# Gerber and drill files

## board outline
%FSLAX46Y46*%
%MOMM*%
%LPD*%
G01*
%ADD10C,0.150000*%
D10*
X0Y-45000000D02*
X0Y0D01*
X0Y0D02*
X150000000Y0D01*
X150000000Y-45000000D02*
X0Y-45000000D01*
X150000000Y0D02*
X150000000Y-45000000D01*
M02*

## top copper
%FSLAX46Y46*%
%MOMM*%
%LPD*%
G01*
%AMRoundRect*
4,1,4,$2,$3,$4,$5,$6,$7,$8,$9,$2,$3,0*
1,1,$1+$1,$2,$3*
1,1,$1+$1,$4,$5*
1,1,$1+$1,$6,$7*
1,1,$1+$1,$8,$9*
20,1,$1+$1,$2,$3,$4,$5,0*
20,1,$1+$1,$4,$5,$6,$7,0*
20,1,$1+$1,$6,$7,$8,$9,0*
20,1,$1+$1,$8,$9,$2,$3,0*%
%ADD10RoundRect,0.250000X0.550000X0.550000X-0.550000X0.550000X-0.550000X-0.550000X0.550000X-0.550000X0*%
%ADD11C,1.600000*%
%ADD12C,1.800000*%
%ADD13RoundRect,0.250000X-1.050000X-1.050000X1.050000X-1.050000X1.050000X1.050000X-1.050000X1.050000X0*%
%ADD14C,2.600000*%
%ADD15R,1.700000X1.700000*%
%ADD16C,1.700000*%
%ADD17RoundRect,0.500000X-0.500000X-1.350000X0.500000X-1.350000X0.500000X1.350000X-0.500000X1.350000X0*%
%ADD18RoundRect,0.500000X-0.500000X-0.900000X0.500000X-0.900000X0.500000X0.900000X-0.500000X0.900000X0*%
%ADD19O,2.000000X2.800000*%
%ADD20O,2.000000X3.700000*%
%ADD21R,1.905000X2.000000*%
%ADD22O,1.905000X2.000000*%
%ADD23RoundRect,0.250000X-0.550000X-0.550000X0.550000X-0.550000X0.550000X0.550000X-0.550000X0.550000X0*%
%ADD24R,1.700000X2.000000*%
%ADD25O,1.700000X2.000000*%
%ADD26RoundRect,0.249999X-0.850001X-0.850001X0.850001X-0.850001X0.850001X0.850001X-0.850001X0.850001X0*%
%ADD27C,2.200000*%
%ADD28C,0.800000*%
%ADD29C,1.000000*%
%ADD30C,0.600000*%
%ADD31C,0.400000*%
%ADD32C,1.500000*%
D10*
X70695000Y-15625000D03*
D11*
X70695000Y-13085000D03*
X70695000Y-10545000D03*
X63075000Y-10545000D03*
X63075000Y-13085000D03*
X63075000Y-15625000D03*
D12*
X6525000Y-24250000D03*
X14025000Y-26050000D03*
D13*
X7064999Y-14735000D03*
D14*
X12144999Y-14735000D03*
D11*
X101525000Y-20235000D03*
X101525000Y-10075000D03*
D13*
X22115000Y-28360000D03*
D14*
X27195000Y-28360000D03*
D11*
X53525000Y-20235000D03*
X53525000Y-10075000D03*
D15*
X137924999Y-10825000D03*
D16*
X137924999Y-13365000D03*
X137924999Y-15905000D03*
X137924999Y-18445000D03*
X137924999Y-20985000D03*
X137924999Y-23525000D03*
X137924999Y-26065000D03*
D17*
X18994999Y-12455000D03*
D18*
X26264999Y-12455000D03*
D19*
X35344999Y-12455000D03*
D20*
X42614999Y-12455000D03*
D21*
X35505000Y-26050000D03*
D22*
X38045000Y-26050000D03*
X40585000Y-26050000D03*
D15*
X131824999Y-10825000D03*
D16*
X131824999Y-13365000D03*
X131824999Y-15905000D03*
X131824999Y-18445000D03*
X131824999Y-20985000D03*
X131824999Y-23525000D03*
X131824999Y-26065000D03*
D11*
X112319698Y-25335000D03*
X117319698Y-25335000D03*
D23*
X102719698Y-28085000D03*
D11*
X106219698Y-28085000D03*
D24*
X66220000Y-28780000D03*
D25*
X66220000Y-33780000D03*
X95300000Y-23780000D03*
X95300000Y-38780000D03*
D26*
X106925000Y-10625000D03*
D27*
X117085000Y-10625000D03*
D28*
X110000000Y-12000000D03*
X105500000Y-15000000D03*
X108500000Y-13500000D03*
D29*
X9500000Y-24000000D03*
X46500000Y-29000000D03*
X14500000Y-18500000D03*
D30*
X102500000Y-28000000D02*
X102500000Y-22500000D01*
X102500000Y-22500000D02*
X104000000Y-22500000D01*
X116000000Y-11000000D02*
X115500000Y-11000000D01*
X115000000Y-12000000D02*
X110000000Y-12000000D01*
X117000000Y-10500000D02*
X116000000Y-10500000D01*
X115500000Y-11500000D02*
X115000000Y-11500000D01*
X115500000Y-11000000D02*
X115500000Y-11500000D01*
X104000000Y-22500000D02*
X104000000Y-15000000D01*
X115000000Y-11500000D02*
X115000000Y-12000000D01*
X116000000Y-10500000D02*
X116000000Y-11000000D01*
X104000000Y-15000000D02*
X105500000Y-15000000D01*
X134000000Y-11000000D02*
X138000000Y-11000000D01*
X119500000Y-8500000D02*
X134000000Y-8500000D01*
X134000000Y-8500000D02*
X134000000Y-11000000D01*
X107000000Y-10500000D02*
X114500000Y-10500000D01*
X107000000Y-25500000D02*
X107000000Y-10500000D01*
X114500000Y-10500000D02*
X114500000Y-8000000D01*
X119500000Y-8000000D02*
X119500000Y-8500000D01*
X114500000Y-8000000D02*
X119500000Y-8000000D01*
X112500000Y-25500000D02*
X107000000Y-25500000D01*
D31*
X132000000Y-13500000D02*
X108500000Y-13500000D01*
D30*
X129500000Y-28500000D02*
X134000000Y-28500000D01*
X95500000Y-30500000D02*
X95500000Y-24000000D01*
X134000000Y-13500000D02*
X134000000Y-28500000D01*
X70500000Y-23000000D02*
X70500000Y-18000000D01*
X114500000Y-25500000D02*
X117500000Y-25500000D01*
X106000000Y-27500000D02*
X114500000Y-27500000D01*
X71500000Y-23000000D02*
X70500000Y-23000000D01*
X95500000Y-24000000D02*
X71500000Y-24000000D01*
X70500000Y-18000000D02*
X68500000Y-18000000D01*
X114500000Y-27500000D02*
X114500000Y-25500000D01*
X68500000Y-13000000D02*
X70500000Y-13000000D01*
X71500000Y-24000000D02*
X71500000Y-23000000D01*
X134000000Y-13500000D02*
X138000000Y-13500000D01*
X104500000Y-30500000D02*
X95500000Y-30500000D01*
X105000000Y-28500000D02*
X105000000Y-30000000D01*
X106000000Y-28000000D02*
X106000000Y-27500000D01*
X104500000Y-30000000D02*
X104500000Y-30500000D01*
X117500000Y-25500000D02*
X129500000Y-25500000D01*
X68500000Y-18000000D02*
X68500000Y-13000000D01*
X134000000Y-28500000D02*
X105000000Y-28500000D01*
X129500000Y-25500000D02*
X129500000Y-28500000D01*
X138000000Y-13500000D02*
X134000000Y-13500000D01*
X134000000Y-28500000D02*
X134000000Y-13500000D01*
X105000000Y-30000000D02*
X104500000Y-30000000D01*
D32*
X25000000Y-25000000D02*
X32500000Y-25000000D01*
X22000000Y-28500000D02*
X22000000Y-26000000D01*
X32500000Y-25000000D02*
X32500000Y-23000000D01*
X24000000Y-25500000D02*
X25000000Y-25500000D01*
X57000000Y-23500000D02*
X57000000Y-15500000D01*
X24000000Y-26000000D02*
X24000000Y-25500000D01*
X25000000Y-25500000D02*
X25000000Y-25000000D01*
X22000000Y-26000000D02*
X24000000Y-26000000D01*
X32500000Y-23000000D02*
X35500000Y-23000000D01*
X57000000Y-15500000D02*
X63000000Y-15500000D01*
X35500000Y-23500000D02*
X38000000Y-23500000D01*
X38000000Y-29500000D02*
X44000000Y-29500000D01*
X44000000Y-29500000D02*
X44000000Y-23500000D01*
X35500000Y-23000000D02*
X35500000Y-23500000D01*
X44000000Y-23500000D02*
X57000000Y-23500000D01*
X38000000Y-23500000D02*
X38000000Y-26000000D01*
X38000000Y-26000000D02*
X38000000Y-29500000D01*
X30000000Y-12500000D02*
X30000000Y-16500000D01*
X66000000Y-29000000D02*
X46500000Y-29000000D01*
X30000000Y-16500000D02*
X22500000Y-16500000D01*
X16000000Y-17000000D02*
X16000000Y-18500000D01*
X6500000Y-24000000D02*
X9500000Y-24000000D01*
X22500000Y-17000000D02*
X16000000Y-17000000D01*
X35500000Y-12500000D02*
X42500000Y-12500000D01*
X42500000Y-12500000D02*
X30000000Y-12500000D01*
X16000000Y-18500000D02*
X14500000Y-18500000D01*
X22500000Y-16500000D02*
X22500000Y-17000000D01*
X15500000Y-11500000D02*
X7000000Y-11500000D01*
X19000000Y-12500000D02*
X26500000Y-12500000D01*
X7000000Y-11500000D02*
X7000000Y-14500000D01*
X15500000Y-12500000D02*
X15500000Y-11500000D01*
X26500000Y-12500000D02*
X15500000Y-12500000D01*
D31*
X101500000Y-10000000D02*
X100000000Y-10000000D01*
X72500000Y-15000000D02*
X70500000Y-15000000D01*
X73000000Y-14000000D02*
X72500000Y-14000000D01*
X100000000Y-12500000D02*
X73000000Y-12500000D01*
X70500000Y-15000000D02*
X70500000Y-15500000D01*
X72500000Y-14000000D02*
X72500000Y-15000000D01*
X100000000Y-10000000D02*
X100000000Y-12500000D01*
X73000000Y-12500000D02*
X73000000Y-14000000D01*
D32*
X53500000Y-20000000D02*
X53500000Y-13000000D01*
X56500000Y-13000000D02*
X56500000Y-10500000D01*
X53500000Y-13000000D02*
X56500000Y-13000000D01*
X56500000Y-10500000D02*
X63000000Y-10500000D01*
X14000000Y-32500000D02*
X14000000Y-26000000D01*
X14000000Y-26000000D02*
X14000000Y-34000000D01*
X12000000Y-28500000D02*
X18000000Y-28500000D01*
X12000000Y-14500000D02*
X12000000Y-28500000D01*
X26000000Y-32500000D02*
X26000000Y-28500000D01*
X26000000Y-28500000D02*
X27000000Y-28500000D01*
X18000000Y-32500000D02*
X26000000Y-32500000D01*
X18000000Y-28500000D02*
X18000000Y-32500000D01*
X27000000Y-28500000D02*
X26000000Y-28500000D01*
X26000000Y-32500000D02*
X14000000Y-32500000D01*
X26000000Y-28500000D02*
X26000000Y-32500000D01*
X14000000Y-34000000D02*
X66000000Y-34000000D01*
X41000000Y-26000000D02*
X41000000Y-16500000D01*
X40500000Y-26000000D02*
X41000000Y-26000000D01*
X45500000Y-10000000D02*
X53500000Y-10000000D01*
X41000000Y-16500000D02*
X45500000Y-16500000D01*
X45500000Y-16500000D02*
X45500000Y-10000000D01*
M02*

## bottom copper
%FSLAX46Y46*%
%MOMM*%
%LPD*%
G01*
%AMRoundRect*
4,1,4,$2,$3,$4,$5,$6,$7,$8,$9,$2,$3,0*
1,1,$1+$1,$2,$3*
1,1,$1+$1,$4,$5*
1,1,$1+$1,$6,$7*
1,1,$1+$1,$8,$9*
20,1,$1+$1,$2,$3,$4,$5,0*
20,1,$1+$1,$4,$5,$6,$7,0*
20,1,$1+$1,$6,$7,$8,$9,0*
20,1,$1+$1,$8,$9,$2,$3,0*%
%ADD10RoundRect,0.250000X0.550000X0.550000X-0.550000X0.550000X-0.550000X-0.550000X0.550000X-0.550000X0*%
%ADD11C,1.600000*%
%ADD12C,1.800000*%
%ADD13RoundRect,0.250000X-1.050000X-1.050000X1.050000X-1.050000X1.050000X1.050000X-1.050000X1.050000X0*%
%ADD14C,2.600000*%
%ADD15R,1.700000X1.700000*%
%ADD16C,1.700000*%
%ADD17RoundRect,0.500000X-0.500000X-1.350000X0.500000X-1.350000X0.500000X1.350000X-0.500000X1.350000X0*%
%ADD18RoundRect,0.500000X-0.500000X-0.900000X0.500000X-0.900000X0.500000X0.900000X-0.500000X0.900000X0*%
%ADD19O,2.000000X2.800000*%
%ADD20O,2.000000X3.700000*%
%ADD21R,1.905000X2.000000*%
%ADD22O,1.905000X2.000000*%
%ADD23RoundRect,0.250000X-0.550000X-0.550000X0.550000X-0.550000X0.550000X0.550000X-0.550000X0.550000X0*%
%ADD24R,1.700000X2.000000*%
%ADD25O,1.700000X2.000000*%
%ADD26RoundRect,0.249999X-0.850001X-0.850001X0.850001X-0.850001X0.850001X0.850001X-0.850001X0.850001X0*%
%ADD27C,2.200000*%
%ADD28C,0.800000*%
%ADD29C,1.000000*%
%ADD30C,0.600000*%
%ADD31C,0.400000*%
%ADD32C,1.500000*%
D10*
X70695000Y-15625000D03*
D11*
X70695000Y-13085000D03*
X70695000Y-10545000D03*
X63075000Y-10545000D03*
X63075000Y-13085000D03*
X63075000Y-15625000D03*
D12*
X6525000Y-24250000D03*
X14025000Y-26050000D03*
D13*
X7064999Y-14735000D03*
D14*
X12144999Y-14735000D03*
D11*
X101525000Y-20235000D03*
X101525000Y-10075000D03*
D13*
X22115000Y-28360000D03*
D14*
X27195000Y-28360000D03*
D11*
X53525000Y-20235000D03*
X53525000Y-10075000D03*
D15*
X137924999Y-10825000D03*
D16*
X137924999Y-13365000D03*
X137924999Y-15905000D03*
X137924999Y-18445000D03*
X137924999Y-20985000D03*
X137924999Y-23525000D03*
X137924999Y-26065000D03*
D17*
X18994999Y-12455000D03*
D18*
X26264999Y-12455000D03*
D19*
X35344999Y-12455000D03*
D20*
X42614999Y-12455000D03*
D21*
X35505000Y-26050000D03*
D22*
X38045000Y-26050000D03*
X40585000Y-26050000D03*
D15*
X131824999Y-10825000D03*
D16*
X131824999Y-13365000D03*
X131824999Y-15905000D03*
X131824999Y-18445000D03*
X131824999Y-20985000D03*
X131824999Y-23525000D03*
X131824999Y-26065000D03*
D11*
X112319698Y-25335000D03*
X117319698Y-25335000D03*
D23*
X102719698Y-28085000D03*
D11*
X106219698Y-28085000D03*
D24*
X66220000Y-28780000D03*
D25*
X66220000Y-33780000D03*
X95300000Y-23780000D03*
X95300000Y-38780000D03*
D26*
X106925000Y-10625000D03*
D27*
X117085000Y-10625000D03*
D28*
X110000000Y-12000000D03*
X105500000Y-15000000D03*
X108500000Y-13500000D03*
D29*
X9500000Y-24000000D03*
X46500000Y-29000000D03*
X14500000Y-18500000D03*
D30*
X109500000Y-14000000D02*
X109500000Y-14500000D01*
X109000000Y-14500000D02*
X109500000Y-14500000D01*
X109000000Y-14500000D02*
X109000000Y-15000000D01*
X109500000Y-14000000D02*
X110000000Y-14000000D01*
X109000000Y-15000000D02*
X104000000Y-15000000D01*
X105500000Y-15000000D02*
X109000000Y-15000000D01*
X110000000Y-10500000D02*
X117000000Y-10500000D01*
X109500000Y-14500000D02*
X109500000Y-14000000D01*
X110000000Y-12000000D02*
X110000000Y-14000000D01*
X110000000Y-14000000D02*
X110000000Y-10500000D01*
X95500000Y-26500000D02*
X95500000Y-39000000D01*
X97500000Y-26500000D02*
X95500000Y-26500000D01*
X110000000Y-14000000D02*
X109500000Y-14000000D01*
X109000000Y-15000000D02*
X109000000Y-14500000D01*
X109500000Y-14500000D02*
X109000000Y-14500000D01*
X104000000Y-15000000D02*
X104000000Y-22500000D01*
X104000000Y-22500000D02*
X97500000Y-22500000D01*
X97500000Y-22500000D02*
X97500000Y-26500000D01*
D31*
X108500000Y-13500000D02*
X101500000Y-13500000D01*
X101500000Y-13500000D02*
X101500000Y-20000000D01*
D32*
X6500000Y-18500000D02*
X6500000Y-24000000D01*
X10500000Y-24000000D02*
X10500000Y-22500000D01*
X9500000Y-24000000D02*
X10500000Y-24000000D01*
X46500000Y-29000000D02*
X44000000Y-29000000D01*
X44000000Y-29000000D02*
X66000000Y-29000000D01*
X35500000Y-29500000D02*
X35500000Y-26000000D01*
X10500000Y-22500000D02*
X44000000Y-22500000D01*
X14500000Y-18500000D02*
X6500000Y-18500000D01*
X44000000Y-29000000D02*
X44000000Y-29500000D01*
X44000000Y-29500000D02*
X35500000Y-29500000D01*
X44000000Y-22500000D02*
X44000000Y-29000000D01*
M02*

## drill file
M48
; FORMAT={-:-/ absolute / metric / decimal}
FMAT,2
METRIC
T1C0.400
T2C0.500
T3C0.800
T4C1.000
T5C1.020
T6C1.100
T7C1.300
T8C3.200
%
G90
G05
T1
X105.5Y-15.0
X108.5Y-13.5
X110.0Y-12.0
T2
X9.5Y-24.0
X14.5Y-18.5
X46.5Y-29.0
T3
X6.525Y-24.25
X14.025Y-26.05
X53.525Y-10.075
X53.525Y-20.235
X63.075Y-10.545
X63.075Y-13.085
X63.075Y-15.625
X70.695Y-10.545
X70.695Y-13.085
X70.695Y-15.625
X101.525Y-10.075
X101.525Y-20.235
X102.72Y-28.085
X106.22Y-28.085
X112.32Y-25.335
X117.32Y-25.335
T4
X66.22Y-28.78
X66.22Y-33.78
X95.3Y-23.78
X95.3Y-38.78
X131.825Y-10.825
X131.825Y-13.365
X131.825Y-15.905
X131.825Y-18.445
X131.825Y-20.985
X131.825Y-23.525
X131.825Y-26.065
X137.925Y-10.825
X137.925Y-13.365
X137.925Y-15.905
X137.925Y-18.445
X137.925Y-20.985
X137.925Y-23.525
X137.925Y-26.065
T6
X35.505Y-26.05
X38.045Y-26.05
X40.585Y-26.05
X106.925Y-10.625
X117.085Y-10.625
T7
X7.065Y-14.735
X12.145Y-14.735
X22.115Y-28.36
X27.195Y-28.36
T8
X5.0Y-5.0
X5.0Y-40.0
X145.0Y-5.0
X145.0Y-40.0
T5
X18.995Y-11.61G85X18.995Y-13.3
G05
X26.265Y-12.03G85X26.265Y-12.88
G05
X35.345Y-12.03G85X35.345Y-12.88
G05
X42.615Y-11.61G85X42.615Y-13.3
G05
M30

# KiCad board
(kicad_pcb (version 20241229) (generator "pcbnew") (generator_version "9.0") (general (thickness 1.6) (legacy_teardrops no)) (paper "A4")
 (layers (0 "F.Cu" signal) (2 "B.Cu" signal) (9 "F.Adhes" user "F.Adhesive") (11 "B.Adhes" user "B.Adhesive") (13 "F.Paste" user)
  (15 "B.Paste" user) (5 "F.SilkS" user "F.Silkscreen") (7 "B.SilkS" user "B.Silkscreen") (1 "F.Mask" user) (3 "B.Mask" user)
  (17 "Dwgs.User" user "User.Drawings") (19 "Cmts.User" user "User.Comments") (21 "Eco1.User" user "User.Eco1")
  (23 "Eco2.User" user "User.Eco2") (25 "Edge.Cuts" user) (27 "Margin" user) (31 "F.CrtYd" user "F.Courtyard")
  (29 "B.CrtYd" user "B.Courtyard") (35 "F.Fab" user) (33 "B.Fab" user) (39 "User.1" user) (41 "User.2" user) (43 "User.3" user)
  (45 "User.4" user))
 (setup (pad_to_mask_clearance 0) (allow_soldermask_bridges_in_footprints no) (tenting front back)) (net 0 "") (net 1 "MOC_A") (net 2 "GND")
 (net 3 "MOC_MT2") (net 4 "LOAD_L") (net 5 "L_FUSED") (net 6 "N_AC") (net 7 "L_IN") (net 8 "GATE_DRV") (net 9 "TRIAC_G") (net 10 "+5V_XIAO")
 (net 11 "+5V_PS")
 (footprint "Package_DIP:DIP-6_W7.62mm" (layer "F.Cu") (at 70.695 15.625 180)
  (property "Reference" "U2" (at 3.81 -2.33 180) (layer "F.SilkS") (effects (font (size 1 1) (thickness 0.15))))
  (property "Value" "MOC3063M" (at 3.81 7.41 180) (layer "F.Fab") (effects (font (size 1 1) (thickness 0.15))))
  (pad "1" thru_hole roundrect (at 0 0 180) (size 1.6 1.6) (drill 0.8) (layers "*.Cu" "*.Mask") (remove_unused_layers no)
   (roundrect_rratio 0.15625) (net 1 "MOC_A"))
  (pad "2" thru_hole circle (at 0 2.54 180) (size 1.6 1.6) (drill 0.8) (layers "*.Cu" "*.Mask") (remove_unused_layers no) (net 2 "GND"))
  (pad "3" thru_hole circle (at 0 5.08 180) (size 1.6 1.6) (drill 0.8) (layers "*.Cu" "*.Mask") (remove_unused_layers no))
  (pad "4" thru_hole circle (at 7.62 5.08 180) (size 1.6 1.6) (drill 0.8) (layers "*.Cu" "*.Mask") (remove_unused_layers no)
   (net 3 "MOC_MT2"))
  (pad "5" thru_hole circle (at 7.62 2.54 180) (size 1.6 1.6) (drill 0.8) (layers "*.Cu" "*.Mask") (remove_unused_layers no))
  (pad "6" thru_hole circle (at 7.62 0 180) (size 1.6 1.6) (drill 0.8) (layers "*.Cu" "*.Mask") (remove_unused_layers no) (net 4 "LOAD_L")))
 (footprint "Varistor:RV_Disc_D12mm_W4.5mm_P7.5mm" (layer "F.Cu") (at 6.525 24.25)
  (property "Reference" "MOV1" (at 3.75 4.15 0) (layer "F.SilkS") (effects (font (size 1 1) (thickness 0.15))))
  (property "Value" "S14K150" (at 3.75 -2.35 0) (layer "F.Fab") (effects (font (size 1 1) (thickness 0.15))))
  (pad "1" thru_hole circle (at 0 0) (size 1.8 1.8) (drill 0.8) (layers "*.Cu" "*.Mask") (remove_unused_layers no) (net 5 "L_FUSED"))
  (pad "2" thru_hole circle (at 7.5 1.8) (size 1.8 1.8) (drill 0.8) (layers "*.Cu" "*.Mask") (remove_unused_layers no) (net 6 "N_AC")))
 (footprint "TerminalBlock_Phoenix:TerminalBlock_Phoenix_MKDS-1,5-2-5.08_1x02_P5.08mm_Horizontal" (layer "F.Cu") (at 7.064999 14.735)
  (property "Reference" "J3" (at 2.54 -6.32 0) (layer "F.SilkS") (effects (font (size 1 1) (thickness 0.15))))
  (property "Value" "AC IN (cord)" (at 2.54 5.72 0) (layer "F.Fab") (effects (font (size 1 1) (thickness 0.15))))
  (pad "1" thru_hole roundrect (at 0 0) (size 2.6 2.6) (drill 1.3) (layers "*.Cu" "*.Mask") (remove_unused_layers no)
   (roundrect_rratio 0.096154) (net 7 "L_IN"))
  (pad "2" thru_hole circle (at 5.08 0) (size 2.6 2.6) (drill 1.3) (layers "*.Cu" "*.Mask") (remove_unused_layers no) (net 6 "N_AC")))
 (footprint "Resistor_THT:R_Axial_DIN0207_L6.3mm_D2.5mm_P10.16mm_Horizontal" (layer "F.Cu") (at 101.525 20.235 90)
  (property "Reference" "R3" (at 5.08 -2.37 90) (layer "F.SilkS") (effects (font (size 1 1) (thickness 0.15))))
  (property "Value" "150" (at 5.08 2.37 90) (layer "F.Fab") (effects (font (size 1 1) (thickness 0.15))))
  (pad "1" thru_hole circle (at 0 0 90) (size 1.6 1.6) (drill 0.8) (layers "*.Cu" "*.Mask") (remove_unused_layers no) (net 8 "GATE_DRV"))
  (pad "2" thru_hole circle (at 10.16 0 90) (size 1.6 1.6) (drill 0.8) (layers "*.Cu" "*.Mask") (remove_unused_layers no) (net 1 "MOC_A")))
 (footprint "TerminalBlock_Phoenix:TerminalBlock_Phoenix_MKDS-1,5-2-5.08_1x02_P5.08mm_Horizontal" (layer "F.Cu") (at 22.115 28.36)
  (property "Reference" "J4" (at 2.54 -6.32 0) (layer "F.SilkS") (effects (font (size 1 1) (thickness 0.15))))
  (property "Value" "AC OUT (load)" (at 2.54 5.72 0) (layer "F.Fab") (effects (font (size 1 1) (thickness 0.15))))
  (pad "1" thru_hole roundrect (at 0 0) (size 2.6 2.6) (drill 1.3) (layers "*.Cu" "*.Mask") (remove_unused_layers no)
   (roundrect_rratio 0.096154) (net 4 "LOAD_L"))
  (pad "2" thru_hole circle (at 5.08 0) (size 2.6 2.6) (drill 1.3) (layers "*.Cu" "*.Mask") (remove_unused_layers no) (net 6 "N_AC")))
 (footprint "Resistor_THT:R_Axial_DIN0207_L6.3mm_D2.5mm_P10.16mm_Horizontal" (layer "F.Cu") (at 53.525 20.235 90)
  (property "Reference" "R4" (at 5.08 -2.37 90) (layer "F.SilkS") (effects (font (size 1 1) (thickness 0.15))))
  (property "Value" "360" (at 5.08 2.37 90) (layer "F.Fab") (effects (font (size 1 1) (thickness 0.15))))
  (pad "1" thru_hole circle (at 0 0 90) (size 1.6 1.6) (drill 0.8) (layers "*.Cu" "*.Mask") (remove_unused_layers no) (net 3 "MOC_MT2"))
  (pad "2" thru_hole circle (at 10.16 0 90) (size 1.6 1.6) (drill 0.8) (layers "*.Cu" "*.Mask") (remove_unused_layers no) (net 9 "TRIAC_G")))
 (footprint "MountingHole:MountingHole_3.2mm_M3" (layer "F.Cu") (at 145 5)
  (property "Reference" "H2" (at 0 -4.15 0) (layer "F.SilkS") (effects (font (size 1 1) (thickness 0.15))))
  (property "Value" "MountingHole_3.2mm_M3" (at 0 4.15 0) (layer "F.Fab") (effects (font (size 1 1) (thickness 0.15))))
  (pad "" np_thru_hole circle (at 0 0) (size 3.2 3.2) (drill 3.2) (layers "*.Cu" "*.Mask")))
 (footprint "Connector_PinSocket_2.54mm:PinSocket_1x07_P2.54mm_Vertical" (layer "F.Cu") (at 137.924999 10.825)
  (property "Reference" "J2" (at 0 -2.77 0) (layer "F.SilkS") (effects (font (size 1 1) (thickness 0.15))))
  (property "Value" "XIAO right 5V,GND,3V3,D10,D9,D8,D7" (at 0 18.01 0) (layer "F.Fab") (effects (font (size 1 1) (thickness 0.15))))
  (pad "1" thru_hole rect (at 0 0) (size 1.7 1.7) (drill 1) (layers "*.Cu" "*.Mask") (remove_unused_layers no) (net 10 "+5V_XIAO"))
  (pad "2" thru_hole circle (at 0 2.54) (size 1.7 1.7) (drill 1) (layers "*.Cu" "*.Mask") (remove_unused_layers no) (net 2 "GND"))
  (pad "3" thru_hole circle (at 0 5.08) (size 1.7 1.7) (drill 1) (layers "*.Cu" "*.Mask") (remove_unused_layers no))
  (pad "4" thru_hole circle (at 0 7.62) (size 1.7 1.7) (drill 1) (layers "*.Cu" "*.Mask") (remove_unused_layers no))
  (pad "5" thru_hole circle (at 0 10.16) (size 1.7 1.7) (drill 1) (layers "*.Cu" "*.Mask") (remove_unused_layers no))
  (pad "6" thru_hole circle (at 0 12.7) (size 1.7 1.7) (drill 1) (layers "*.Cu" "*.Mask") (remove_unused_layers no))
  (pad "7" thru_hole circle (at 0 15.24) (size 1.7 1.7) (drill 1) (layers "*.Cu" "*.Mask") (remove_unused_layers no)))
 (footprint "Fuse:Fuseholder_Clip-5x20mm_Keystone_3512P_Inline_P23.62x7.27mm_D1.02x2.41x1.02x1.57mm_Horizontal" (layer "F.Cu")
  (at 18.994999 12.455)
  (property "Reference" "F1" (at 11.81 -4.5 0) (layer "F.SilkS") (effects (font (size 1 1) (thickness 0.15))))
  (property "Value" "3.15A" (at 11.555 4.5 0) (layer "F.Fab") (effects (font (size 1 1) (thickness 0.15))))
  (pad "1" thru_hole roundrect (at 0 0) (size 2 3.7) (drill oval 1.02 2.71) (layers "*.Cu" "*.Mask") (remove_unused_layers no)
   (roundrect_rratio 0.25) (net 7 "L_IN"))
  (pad "1" thru_hole roundrect (at 7.27 0) (size 2 2.8) (drill oval 1.02 1.87) (layers "*.Cu" "*.Mask") (remove_unused_layers no)
   (roundrect_rratio 0.25) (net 7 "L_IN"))
  (pad "2" thru_hole oval (at 16.35 0) (size 2 2.8) (drill oval 1.02 1.87) (layers "*.Cu" "*.Mask") (remove_unused_layers no)
   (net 5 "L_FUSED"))
  (pad "2" thru_hole oval (at 23.62 0) (size 2 3.7) (drill oval 1.02 2.71) (layers "*.Cu" "*.Mask") (remove_unused_layers no)
   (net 5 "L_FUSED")))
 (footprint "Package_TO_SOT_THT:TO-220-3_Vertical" (layer "F.Cu") (at 35.505 26.05)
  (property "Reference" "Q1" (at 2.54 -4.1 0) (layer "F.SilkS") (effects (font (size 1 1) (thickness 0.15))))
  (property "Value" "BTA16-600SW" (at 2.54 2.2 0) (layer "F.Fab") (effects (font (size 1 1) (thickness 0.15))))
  (pad "1" thru_hole rect (at 0 0) (size 1.905 2) (drill 1.1) (layers "*.Cu" "*.Mask") (remove_unused_layers no) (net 5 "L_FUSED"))
  (pad "2" thru_hole oval (at 2.54 0) (size 1.905 2) (drill 1.1) (layers "*.Cu" "*.Mask") (remove_unused_layers no) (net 4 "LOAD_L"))
  (pad "3" thru_hole oval (at 5.08 0) (size 1.905 2) (drill 1.1) (layers "*.Cu" "*.Mask") (remove_unused_layers no) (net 9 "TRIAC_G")))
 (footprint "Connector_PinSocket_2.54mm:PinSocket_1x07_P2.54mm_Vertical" (layer "F.Cu") (at 131.824999 10.825)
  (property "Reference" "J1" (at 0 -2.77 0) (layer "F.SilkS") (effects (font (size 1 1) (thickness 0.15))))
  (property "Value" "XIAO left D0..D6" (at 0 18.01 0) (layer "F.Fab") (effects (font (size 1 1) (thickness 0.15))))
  (pad "1" thru_hole rect (at 0 0) (size 1.7 1.7) (drill 1) (layers "*.Cu" "*.Mask") (remove_unused_layers no))
  (pad "2" thru_hole circle (at 0 2.54) (size 1.7 1.7) (drill 1) (layers "*.Cu" "*.Mask") (remove_unused_layers no) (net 8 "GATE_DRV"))
  (pad "3" thru_hole circle (at 0 5.08) (size 1.7 1.7) (drill 1) (layers "*.Cu" "*.Mask") (remove_unused_layers no))
  (pad "4" thru_hole circle (at 0 7.62) (size 1.7 1.7) (drill 1) (layers "*.Cu" "*.Mask") (remove_unused_layers no))
  (pad "5" thru_hole circle (at 0 10.16) (size 1.7 1.7) (drill 1) (layers "*.Cu" "*.Mask") (remove_unused_layers no))
  (pad "6" thru_hole circle (at 0 12.7) (size 1.7 1.7) (drill 1) (layers "*.Cu" "*.Mask") (remove_unused_layers no))
  (pad "7" thru_hole circle (at 0 15.24) (size 1.7 1.7) (drill 1) (layers "*.Cu" "*.Mask") (remove_unused_layers no)))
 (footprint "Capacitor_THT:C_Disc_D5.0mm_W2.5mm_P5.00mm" (layer "F.Cu") (at 112.319698 25.335)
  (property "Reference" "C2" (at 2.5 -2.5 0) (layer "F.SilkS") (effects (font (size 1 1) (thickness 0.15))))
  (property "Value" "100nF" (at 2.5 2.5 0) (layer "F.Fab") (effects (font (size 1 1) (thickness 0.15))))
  (pad "1" thru_hole circle (at 0 0) (size 1.6 1.6) (drill 0.8) (layers "*.Cu" "*.Mask") (remove_unused_layers no) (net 10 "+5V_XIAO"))
  (pad "2" thru_hole circle (at 5 0) (size 1.6 1.6) (drill 0.8) (layers "*.Cu" "*.Mask") (remove_unused_layers no) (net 2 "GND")))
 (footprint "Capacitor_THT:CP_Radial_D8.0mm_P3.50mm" (layer "F.Cu") (at 102.719698 28.085)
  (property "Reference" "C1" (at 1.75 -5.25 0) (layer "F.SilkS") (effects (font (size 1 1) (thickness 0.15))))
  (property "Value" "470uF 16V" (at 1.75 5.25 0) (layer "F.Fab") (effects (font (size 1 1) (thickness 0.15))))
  (pad "1" thru_hole roundrect (at 0 0) (size 1.6 1.6) (drill 0.8) (layers "*.Cu" "*.Mask") (remove_unused_layers no)
   (roundrect_rratio 0.15625) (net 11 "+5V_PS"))
  (pad "2" thru_hole circle (at 3.5 0) (size 1.6 1.6) (drill 0.8) (layers "*.Cu" "*.Mask") (remove_unused_layers no) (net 2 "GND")))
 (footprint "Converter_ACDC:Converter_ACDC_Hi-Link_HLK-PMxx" (layer "F.Cu") (at 66.22 28.78)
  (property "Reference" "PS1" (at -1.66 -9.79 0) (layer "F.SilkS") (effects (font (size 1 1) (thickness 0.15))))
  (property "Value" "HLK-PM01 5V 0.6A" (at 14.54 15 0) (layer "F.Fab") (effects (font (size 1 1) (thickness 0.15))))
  (pad "1" thru_hole rect (at 0 0) (size 1.7 2) (drill 1) (layers "*.Cu" "*.Mask") (remove_unused_layers no) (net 5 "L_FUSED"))
  (pad "2" thru_hole oval (at 0 5) (size 1.7 2) (drill 1) (layers "*.Cu" "*.Mask") (remove_unused_layers no) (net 6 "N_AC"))
  (pad "3" thru_hole oval (at 29.08 -5) (size 1.7 2) (drill 1) (layers "*.Cu" "*.Mask") (remove_unused_layers no) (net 2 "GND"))
  (pad "4" thru_hole oval (at 29.08 10) (size 1.7 2) (drill 1) (layers "*.Cu" "*.Mask") (remove_unused_layers no) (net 11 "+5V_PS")))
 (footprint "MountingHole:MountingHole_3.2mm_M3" (layer "F.Cu") (at 5 40)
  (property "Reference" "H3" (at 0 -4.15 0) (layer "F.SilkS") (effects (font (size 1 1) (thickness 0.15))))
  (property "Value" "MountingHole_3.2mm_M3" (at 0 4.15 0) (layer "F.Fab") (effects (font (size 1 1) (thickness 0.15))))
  (pad "" np_thru_hole circle (at 0 0) (size 3.2 3.2) (drill 3.2) (layers "*.Cu" "*.Mask")))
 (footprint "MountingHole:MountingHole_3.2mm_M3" (layer "F.Cu") (at 5 5)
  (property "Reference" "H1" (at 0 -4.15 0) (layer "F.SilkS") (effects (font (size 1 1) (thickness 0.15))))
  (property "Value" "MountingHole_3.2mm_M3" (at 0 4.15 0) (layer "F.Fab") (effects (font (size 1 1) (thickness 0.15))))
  (pad "" np_thru_hole circle (at 0 0) (size 3.2 3.2) (drill 3.2) (layers "*.Cu" "*.Mask")))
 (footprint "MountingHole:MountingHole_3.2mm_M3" (layer "F.Cu") (at 145 40)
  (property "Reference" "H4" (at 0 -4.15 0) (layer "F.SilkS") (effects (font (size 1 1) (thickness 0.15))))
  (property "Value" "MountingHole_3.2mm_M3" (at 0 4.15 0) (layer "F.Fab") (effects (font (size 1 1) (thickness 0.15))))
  (pad "" np_thru_hole circle (at 0 0) (size 3.2 3.2) (drill 3.2) (layers "*.Cu" "*.Mask")))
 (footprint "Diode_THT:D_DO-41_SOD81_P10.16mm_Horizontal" (layer "F.Cu") (at 106.925 10.625)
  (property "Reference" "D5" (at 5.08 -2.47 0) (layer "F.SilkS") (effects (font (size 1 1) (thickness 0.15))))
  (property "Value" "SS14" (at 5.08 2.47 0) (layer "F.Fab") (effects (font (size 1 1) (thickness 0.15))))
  (pad "1" thru_hole roundrect (at 0 0) (size 2.2 2.2) (drill 1.1) (layers "*.Cu" "*.Mask") (remove_unused_layers no)
   (roundrect_rratio 0.113636) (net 10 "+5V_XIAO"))
  (pad "2" thru_hole circle (at 10.16 0) (size 2.2 2.2) (drill 1.1) (layers "*.Cu" "*.Mask") (remove_unused_layers no) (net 11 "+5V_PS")))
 (gr_line (start 0 45) (end 0 0) (stroke (width 0.15) (type default)) (layer "Edge.Cuts"))
 (gr_line (start 0 0) (end 150 0) (stroke (width 0.15) (type default)) (layer "Edge.Cuts"))
 (gr_line (start 150 45) (end 0 45) (stroke (width 0.15) (type default)) (layer "Edge.Cuts"))
 (gr_line (start 150 0) (end 150 45) (stroke (width 0.15) (type default)) (layer "Edge.Cuts"))
 (segment (start 102.5 28) (end 102.5 22.5) (width 0.6) (layer "F.Cu") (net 11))
 (segment (start 102.5 22.5) (end 104 22.5) (width 0.6) (layer "F.Cu") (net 11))
 (segment (start 116 11) (end 115.5 11) (width 0.6) (layer "F.Cu") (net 11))
 (segment (start 115 12) (end 110 12) (width 0.6) (layer "F.Cu") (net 11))
 (segment (start 117 10.5) (end 116 10.5) (width 0.6) (layer "F.Cu") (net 11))
 (segment (start 115.5 11.5) (end 115 11.5) (width 0.6) (layer "F.Cu") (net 11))
 (segment (start 115.5 11) (end 115.5 11.5) (width 0.6) (layer "F.Cu") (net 11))
 (segment (start 104 22.5) (end 104 15) (width 0.6) (layer "F.Cu") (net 11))
 (segment (start 115 11.5) (end 115 12) (width 0.6) (layer "F.Cu") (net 11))
 (segment (start 116 10.5) (end 116 11) (width 0.6) (layer "F.Cu") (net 11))
 (segment (start 104 15) (end 105.5 15) (width 0.6) (layer "F.Cu") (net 11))
 (via (at 110 12) (size 0.8) (drill 0.4) (layers "F.Cu" "B.Cu") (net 11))
 (via (at 105.5 15) (size 0.8) (drill 0.4) (layers "F.Cu" "B.Cu") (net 11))
 (segment (start 109.5 14) (end 109.5 14.5) (width 0.6) (layer "B.Cu") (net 11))
 (segment (start 109 14.5) (end 109.5 14.5) (width 0.6) (layer "B.Cu") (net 11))
 (segment (start 109 14.5) (end 109 15) (width 0.6) (layer "B.Cu") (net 11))
 (segment (start 109.5 14) (end 110 14) (width 0.6) (layer "B.Cu") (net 11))
 (segment (start 109 15) (end 104 15) (width 0.6) (layer "B.Cu") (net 11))
 (segment (start 105.5 15) (end 109 15) (width 0.6) (layer "B.Cu") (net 11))
 (segment (start 110 10.5) (end 117 10.5) (width 0.6) (layer "B.Cu") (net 11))
 (segment (start 109.5 14.5) (end 109.5 14) (width 0.6) (layer "B.Cu") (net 11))
 (segment (start 110 12) (end 110 14) (width 0.6) (layer "B.Cu") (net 11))
 (segment (start 110 14) (end 110 10.5) (width 0.6) (layer "B.Cu") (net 11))
 (segment (start 95.5 26.5) (end 95.5 39) (width 0.6) (layer "B.Cu") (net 11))
 (segment (start 97.5 26.5) (end 95.5 26.5) (width 0.6) (layer "B.Cu") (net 11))
 (segment (start 110 14) (end 109.5 14) (width 0.6) (layer "B.Cu") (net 11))
 (segment (start 109 15) (end 109 14.5) (width 0.6) (layer "B.Cu") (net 11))
 (segment (start 109.5 14.5) (end 109 14.5) (width 0.6) (layer "B.Cu") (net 11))
 (segment (start 104 15) (end 104 22.5) (width 0.6) (layer "B.Cu") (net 11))
 (segment (start 104 22.5) (end 97.5 22.5) (width 0.6) (layer "B.Cu") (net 11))
 (segment (start 97.5 22.5) (end 97.5 26.5) (width 0.6) (layer "B.Cu") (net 11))
 (segment (start 134 11) (end 138 11) (width 0.6) (layer "F.Cu") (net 10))
 (segment (start 119.5 8.5) (end 134 8.5) (width 0.6) (layer "F.Cu") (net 10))
 (segment (start 134 8.5) (end 134 11) (width 0.6) (layer "F.Cu") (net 10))
 (segment (start 107 10.5) (end 114.5 10.5) (width 0.6) (layer "F.Cu") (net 10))
 (segment (start 107 25.5) (end 107 10.5) (width 0.6) (layer "F.Cu") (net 10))
 (segment (start 114.5 10.5) (end 114.5 8) (width 0.6) (layer "F.Cu") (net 10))
 (segment (start 119.5 8) (end 119.5 8.5) (width 0.6) (layer "F.Cu") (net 10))
 (segment (start 114.5 8) (end 119.5 8) (width 0.6) (layer "F.Cu") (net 10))
 (segment (start 112.5 25.5) (end 107 25.5) (width 0.6) (layer "F.Cu") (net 10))
 (segment (start 132 13.5) (end 108.5 13.5) (width 0.4) (layer "F.Cu") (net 8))
 (via (at 108.5 13.5) (size 0.8) (drill 0.4) (layers "F.Cu" "B.Cu") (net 8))
 (segment (start 108.5 13.5) (end 101.5 13.5) (width 0.4) (layer "B.Cu") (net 8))
 (segment (start 101.5 13.5) (end 101.5 20) (width 0.4) (layer "B.Cu") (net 8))
 (segment (start 129.5 28.5) (end 134 28.5) (width 0.6) (layer "F.Cu") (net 2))
 (segment (start 95.5 30.5) (end 95.5 24) (width 0.6) (layer "F.Cu") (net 2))
 (segment (start 134 13.5) (end 134 28.5) (width 0.6) (layer "F.Cu") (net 2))
 (segment (start 70.5 23) (end 70.5 18) (width 0.6) (layer "F.Cu") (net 2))
 (segment (start 114.5 25.5) (end 117.5 25.5) (width 0.6) (layer "F.Cu") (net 2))
 (segment (start 106 27.5) (end 114.5 27.5) (width 0.6) (layer "F.Cu") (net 2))
 (segment (start 71.5 23) (end 70.5 23) (width 0.6) (layer "F.Cu") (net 2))
 (segment (start 95.5 24) (end 71.5 24) (width 0.6) (layer "F.Cu") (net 2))
 (segment (start 70.5 18) (end 68.5 18) (width 0.6) (layer "F.Cu") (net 2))
 (segment (start 114.5 27.5) (end 114.5 25.5) (width 0.6) (layer "F.Cu") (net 2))
 (segment (start 68.5 13) (end 70.5 13) (width 0.6) (layer "F.Cu") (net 2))
 (segment (start 71.5 24) (end 71.5 23) (width 0.6) (layer "F.Cu") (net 2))
 (segment (start 134 13.5) (end 138 13.5) (width 0.6) (layer "F.Cu") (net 2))
 (segment (start 104.5 30.5) (end 95.5 30.5) (width 0.6) (layer "F.Cu") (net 2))
 (segment (start 105 28.5) (end 105 30) (width 0.6) (layer "F.Cu") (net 2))
 (segment (start 106 28) (end 106 27.5) (width 0.6) (layer "F.Cu") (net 2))
 (segment (start 104.5 30) (end 104.5 30.5) (width 0.6) (layer "F.Cu") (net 2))
 (segment (start 117.5 25.5) (end 129.5 25.5) (width 0.6) (layer "F.Cu") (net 2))
 (segment (start 68.5 18) (end 68.5 13) (width 0.6) (layer "F.Cu") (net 2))
 (segment (start 134 28.5) (end 105 28.5) (width 0.6) (layer "F.Cu") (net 2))
 (segment (start 129.5 25.5) (end 129.5 28.5) (width 0.6) (layer "F.Cu") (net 2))
 (segment (start 138 13.5) (end 134 13.5) (width 0.6) (layer "F.Cu") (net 2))
 (segment (start 134 28.5) (end 134 13.5) (width 0.6) (layer "F.Cu") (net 2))
 (segment (start 105 30) (end 104.5 30) (width 0.6) (layer "F.Cu") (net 2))
 (segment (start 25 25) (end 32.5 25) (width 1.5) (layer "F.Cu") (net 4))
 (segment (start 22 28.5) (end 22 26) (width 1.5) (layer "F.Cu") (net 4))
 (segment (start 32.5 25) (end 32.5 23) (width 1.5) (layer "F.Cu") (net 4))
 (segment (start 24 25.5) (end 25 25.5) (width 1.5) (layer "F.Cu") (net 4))
 (segment (start 57 23.5) (end 57 15.5) (width 1.5) (layer "F.Cu") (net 4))
 (segment (start 24 26) (end 24 25.5) (width 1.5) (layer "F.Cu") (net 4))
 (segment (start 25 25.5) (end 25 25) (width 1.5) (layer "F.Cu") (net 4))
 (segment (start 22 26) (end 24 26) (width 1.5) (layer "F.Cu") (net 4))
 (segment (start 32.5 23) (end 35.5 23) (width 1.5) (layer "F.Cu") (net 4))
 (segment (start 57 15.5) (end 63 15.5) (width 1.5) (layer "F.Cu") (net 4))
 (segment (start 35.5 23.5) (end 38 23.5) (width 1.5) (layer "F.Cu") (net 4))
 (segment (start 38 29.5) (end 44 29.5) (width 1.5) (layer "F.Cu") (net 4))
 (segment (start 44 29.5) (end 44 23.5) (width 1.5) (layer "F.Cu") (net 4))
 (segment (start 35.5 23) (end 35.5 23.5) (width 1.5) (layer "F.Cu") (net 4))
 (segment (start 44 23.5) (end 57 23.5) (width 1.5) (layer "F.Cu") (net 4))
 (segment (start 38 23.5) (end 38 26) (width 1.5) (layer "F.Cu") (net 4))
 (segment (start 38 26) (end 38 29.5) (width 1.5) (layer "F.Cu") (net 4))
 (segment (start 30 12.5) (end 30 16.5) (width 1.5) (layer "F.Cu") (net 5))
 (segment (start 66 29) (end 46.5 29) (width 1.5) (layer "F.Cu") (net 5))
 (segment (start 30 16.5) (end 22.5 16.5) (width 1.5) (layer "F.Cu") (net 5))
 (segment (start 16 17) (end 16 18.5) (width 1.5) (layer "F.Cu") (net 5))
 (segment (start 6.5 24) (end 9.5 24) (width 1.5) (layer "F.Cu") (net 5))
 (segment (start 22.5 17) (end 16 17) (width 1.5) (layer "F.Cu") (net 5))
 (segment (start 35.5 12.5) (end 42.5 12.5) (width 1.5) (layer "F.Cu") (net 5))
 (segment (start 42.5 12.5) (end 30 12.5) (width 1.5) (layer "F.Cu") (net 5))
 (segment (start 16 18.5) (end 14.5 18.5) (width 1.5) (layer "F.Cu") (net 5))
 (segment (start 22.5 16.5) (end 22.5 17) (width 1.5) (layer "F.Cu") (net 5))
 (via (at 9.5 24) (size 1) (drill 0.5) (layers "F.Cu" "B.Cu") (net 5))
 (via (at 46.5 29) (size 1) (drill 0.5) (layers "F.Cu" "B.Cu") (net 5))
 (via (at 14.5 18.5) (size 1) (drill 0.5) (layers "F.Cu" "B.Cu") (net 5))
 (segment (start 6.5 18.5) (end 6.5 24) (width 1.5) (layer "B.Cu") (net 5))
 (segment (start 10.5 24) (end 10.5 22.5) (width 1.5) (layer "B.Cu") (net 5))
 (segment (start 9.5 24) (end 10.5 24) (width 1.5) (layer "B.Cu") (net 5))
 (segment (start 46.5 29) (end 44 29) (width 1.5) (layer "B.Cu") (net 5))
 (segment (start 44 29) (end 66 29) (width 1.5) (layer "B.Cu") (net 5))
 (segment (start 35.5 29.5) (end 35.5 26) (width 1.5) (layer "B.Cu") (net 5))
 (segment (start 10.5 22.5) (end 44 22.5) (width 1.5) (layer "B.Cu") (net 5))
 (segment (start 14.5 18.5) (end 6.5 18.5) (width 1.5) (layer "B.Cu") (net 5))
 (segment (start 44 29) (end 44 29.5) (width 1.5) (layer "B.Cu") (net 5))
 (segment (start 44 29.5) (end 35.5 29.5) (width 1.5) (layer "B.Cu") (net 5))
 (segment (start 44 22.5) (end 44 29) (width 1.5) (layer "B.Cu") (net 5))
 (segment (start 15.5 11.5) (end 7 11.5) (width 1.5) (layer "F.Cu") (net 7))
 (segment (start 19 12.5) (end 26.5 12.5) (width 1.5) (layer "F.Cu") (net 7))
 (segment (start 7 11.5) (end 7 14.5) (width 1.5) (layer "F.Cu") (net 7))
 (segment (start 15.5 12.5) (end 15.5 11.5) (width 1.5) (layer "F.Cu") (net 7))
 (segment (start 26.5 12.5) (end 15.5 12.5) (width 1.5) (layer "F.Cu") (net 7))
 (segment (start 101.5 10) (end 100 10) (width 0.4) (layer "F.Cu") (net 1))
 (segment (start 72.5 15) (end 70.5 15) (width 0.4) (layer "F.Cu") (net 1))
 (segment (start 73 14) (end 72.5 14) (width 0.4) (layer "F.Cu") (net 1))
 (segment (start 100 12.5) (end 73 12.5) (width 0.4) (layer "F.Cu") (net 1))
 (segment (start 70.5 15) (end 70.5 15.5) (width 0.4) (layer "F.Cu") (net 1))
 (segment (start 72.5 14) (end 72.5 15) (width 0.4) (layer "F.Cu") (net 1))
 (segment (start 100 10) (end 100 12.5) (width 0.4) (layer "F.Cu") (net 1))
 (segment (start 73 12.5) (end 73 14) (width 0.4) (layer "F.Cu") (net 1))
 (segment (start 53.5 20) (end 53.5 13) (width 1.5) (layer "F.Cu") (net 3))
 (segment (start 56.5 13) (end 56.5 10.5) (width 1.5) (layer "F.Cu") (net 3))
 (segment (start 53.5 13) (end 56.5 13) (width 1.5) (layer "F.Cu") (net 3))
 (segment (start 56.5 10.5) (end 63 10.5) (width 1.5) (layer "F.Cu") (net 3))
 (segment (start 14 32.5) (end 14 26) (width 1.5) (layer "F.Cu") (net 6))
 (segment (start 14 26) (end 14 34) (width 1.5) (layer "F.Cu") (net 6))
 (segment (start 12 28.5) (end 18 28.5) (width 1.5) (layer "F.Cu") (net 6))
 (segment (start 12 14.5) (end 12 28.5) (width 1.5) (layer "F.Cu") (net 6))
 (segment (start 26 32.5) (end 26 28.5) (width 1.5) (layer "F.Cu") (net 6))
 (segment (start 26 28.5) (end 27 28.5) (width 1.5) (layer "F.Cu") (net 6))
 (segment (start 18 32.5) (end 26 32.5) (width 1.5) (layer "F.Cu") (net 6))
 (segment (start 18 28.5) (end 18 32.5) (width 1.5) (layer "F.Cu") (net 6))
 (segment (start 27 28.5) (end 26 28.5) (width 1.5) (layer "F.Cu") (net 6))
 (segment (start 26 32.5) (end 14 32.5) (width 1.5) (layer "F.Cu") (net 6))
 (segment (start 26 28.5) (end 26 32.5) (width 1.5) (layer "F.Cu") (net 6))
 (segment (start 14 34) (end 66 34) (width 1.5) (layer "F.Cu") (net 6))
 (segment (start 41 26) (end 41 16.5) (width 1.5) (layer "F.Cu") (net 9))
 (segment (start 40.5 26) (end 41 26) (width 1.5) (layer "F.Cu") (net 9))
 (segment (start 45.5 10) (end 53.5 10) (width 1.5) (layer "F.Cu") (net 9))
 (segment (start 41 16.5) (end 45.5 16.5) (width 1.5) (layer "F.Cu") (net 9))
 (segment (start 45.5 16.5) (end 45.5 10) (width 1.5) (layer "F.Cu") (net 9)))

